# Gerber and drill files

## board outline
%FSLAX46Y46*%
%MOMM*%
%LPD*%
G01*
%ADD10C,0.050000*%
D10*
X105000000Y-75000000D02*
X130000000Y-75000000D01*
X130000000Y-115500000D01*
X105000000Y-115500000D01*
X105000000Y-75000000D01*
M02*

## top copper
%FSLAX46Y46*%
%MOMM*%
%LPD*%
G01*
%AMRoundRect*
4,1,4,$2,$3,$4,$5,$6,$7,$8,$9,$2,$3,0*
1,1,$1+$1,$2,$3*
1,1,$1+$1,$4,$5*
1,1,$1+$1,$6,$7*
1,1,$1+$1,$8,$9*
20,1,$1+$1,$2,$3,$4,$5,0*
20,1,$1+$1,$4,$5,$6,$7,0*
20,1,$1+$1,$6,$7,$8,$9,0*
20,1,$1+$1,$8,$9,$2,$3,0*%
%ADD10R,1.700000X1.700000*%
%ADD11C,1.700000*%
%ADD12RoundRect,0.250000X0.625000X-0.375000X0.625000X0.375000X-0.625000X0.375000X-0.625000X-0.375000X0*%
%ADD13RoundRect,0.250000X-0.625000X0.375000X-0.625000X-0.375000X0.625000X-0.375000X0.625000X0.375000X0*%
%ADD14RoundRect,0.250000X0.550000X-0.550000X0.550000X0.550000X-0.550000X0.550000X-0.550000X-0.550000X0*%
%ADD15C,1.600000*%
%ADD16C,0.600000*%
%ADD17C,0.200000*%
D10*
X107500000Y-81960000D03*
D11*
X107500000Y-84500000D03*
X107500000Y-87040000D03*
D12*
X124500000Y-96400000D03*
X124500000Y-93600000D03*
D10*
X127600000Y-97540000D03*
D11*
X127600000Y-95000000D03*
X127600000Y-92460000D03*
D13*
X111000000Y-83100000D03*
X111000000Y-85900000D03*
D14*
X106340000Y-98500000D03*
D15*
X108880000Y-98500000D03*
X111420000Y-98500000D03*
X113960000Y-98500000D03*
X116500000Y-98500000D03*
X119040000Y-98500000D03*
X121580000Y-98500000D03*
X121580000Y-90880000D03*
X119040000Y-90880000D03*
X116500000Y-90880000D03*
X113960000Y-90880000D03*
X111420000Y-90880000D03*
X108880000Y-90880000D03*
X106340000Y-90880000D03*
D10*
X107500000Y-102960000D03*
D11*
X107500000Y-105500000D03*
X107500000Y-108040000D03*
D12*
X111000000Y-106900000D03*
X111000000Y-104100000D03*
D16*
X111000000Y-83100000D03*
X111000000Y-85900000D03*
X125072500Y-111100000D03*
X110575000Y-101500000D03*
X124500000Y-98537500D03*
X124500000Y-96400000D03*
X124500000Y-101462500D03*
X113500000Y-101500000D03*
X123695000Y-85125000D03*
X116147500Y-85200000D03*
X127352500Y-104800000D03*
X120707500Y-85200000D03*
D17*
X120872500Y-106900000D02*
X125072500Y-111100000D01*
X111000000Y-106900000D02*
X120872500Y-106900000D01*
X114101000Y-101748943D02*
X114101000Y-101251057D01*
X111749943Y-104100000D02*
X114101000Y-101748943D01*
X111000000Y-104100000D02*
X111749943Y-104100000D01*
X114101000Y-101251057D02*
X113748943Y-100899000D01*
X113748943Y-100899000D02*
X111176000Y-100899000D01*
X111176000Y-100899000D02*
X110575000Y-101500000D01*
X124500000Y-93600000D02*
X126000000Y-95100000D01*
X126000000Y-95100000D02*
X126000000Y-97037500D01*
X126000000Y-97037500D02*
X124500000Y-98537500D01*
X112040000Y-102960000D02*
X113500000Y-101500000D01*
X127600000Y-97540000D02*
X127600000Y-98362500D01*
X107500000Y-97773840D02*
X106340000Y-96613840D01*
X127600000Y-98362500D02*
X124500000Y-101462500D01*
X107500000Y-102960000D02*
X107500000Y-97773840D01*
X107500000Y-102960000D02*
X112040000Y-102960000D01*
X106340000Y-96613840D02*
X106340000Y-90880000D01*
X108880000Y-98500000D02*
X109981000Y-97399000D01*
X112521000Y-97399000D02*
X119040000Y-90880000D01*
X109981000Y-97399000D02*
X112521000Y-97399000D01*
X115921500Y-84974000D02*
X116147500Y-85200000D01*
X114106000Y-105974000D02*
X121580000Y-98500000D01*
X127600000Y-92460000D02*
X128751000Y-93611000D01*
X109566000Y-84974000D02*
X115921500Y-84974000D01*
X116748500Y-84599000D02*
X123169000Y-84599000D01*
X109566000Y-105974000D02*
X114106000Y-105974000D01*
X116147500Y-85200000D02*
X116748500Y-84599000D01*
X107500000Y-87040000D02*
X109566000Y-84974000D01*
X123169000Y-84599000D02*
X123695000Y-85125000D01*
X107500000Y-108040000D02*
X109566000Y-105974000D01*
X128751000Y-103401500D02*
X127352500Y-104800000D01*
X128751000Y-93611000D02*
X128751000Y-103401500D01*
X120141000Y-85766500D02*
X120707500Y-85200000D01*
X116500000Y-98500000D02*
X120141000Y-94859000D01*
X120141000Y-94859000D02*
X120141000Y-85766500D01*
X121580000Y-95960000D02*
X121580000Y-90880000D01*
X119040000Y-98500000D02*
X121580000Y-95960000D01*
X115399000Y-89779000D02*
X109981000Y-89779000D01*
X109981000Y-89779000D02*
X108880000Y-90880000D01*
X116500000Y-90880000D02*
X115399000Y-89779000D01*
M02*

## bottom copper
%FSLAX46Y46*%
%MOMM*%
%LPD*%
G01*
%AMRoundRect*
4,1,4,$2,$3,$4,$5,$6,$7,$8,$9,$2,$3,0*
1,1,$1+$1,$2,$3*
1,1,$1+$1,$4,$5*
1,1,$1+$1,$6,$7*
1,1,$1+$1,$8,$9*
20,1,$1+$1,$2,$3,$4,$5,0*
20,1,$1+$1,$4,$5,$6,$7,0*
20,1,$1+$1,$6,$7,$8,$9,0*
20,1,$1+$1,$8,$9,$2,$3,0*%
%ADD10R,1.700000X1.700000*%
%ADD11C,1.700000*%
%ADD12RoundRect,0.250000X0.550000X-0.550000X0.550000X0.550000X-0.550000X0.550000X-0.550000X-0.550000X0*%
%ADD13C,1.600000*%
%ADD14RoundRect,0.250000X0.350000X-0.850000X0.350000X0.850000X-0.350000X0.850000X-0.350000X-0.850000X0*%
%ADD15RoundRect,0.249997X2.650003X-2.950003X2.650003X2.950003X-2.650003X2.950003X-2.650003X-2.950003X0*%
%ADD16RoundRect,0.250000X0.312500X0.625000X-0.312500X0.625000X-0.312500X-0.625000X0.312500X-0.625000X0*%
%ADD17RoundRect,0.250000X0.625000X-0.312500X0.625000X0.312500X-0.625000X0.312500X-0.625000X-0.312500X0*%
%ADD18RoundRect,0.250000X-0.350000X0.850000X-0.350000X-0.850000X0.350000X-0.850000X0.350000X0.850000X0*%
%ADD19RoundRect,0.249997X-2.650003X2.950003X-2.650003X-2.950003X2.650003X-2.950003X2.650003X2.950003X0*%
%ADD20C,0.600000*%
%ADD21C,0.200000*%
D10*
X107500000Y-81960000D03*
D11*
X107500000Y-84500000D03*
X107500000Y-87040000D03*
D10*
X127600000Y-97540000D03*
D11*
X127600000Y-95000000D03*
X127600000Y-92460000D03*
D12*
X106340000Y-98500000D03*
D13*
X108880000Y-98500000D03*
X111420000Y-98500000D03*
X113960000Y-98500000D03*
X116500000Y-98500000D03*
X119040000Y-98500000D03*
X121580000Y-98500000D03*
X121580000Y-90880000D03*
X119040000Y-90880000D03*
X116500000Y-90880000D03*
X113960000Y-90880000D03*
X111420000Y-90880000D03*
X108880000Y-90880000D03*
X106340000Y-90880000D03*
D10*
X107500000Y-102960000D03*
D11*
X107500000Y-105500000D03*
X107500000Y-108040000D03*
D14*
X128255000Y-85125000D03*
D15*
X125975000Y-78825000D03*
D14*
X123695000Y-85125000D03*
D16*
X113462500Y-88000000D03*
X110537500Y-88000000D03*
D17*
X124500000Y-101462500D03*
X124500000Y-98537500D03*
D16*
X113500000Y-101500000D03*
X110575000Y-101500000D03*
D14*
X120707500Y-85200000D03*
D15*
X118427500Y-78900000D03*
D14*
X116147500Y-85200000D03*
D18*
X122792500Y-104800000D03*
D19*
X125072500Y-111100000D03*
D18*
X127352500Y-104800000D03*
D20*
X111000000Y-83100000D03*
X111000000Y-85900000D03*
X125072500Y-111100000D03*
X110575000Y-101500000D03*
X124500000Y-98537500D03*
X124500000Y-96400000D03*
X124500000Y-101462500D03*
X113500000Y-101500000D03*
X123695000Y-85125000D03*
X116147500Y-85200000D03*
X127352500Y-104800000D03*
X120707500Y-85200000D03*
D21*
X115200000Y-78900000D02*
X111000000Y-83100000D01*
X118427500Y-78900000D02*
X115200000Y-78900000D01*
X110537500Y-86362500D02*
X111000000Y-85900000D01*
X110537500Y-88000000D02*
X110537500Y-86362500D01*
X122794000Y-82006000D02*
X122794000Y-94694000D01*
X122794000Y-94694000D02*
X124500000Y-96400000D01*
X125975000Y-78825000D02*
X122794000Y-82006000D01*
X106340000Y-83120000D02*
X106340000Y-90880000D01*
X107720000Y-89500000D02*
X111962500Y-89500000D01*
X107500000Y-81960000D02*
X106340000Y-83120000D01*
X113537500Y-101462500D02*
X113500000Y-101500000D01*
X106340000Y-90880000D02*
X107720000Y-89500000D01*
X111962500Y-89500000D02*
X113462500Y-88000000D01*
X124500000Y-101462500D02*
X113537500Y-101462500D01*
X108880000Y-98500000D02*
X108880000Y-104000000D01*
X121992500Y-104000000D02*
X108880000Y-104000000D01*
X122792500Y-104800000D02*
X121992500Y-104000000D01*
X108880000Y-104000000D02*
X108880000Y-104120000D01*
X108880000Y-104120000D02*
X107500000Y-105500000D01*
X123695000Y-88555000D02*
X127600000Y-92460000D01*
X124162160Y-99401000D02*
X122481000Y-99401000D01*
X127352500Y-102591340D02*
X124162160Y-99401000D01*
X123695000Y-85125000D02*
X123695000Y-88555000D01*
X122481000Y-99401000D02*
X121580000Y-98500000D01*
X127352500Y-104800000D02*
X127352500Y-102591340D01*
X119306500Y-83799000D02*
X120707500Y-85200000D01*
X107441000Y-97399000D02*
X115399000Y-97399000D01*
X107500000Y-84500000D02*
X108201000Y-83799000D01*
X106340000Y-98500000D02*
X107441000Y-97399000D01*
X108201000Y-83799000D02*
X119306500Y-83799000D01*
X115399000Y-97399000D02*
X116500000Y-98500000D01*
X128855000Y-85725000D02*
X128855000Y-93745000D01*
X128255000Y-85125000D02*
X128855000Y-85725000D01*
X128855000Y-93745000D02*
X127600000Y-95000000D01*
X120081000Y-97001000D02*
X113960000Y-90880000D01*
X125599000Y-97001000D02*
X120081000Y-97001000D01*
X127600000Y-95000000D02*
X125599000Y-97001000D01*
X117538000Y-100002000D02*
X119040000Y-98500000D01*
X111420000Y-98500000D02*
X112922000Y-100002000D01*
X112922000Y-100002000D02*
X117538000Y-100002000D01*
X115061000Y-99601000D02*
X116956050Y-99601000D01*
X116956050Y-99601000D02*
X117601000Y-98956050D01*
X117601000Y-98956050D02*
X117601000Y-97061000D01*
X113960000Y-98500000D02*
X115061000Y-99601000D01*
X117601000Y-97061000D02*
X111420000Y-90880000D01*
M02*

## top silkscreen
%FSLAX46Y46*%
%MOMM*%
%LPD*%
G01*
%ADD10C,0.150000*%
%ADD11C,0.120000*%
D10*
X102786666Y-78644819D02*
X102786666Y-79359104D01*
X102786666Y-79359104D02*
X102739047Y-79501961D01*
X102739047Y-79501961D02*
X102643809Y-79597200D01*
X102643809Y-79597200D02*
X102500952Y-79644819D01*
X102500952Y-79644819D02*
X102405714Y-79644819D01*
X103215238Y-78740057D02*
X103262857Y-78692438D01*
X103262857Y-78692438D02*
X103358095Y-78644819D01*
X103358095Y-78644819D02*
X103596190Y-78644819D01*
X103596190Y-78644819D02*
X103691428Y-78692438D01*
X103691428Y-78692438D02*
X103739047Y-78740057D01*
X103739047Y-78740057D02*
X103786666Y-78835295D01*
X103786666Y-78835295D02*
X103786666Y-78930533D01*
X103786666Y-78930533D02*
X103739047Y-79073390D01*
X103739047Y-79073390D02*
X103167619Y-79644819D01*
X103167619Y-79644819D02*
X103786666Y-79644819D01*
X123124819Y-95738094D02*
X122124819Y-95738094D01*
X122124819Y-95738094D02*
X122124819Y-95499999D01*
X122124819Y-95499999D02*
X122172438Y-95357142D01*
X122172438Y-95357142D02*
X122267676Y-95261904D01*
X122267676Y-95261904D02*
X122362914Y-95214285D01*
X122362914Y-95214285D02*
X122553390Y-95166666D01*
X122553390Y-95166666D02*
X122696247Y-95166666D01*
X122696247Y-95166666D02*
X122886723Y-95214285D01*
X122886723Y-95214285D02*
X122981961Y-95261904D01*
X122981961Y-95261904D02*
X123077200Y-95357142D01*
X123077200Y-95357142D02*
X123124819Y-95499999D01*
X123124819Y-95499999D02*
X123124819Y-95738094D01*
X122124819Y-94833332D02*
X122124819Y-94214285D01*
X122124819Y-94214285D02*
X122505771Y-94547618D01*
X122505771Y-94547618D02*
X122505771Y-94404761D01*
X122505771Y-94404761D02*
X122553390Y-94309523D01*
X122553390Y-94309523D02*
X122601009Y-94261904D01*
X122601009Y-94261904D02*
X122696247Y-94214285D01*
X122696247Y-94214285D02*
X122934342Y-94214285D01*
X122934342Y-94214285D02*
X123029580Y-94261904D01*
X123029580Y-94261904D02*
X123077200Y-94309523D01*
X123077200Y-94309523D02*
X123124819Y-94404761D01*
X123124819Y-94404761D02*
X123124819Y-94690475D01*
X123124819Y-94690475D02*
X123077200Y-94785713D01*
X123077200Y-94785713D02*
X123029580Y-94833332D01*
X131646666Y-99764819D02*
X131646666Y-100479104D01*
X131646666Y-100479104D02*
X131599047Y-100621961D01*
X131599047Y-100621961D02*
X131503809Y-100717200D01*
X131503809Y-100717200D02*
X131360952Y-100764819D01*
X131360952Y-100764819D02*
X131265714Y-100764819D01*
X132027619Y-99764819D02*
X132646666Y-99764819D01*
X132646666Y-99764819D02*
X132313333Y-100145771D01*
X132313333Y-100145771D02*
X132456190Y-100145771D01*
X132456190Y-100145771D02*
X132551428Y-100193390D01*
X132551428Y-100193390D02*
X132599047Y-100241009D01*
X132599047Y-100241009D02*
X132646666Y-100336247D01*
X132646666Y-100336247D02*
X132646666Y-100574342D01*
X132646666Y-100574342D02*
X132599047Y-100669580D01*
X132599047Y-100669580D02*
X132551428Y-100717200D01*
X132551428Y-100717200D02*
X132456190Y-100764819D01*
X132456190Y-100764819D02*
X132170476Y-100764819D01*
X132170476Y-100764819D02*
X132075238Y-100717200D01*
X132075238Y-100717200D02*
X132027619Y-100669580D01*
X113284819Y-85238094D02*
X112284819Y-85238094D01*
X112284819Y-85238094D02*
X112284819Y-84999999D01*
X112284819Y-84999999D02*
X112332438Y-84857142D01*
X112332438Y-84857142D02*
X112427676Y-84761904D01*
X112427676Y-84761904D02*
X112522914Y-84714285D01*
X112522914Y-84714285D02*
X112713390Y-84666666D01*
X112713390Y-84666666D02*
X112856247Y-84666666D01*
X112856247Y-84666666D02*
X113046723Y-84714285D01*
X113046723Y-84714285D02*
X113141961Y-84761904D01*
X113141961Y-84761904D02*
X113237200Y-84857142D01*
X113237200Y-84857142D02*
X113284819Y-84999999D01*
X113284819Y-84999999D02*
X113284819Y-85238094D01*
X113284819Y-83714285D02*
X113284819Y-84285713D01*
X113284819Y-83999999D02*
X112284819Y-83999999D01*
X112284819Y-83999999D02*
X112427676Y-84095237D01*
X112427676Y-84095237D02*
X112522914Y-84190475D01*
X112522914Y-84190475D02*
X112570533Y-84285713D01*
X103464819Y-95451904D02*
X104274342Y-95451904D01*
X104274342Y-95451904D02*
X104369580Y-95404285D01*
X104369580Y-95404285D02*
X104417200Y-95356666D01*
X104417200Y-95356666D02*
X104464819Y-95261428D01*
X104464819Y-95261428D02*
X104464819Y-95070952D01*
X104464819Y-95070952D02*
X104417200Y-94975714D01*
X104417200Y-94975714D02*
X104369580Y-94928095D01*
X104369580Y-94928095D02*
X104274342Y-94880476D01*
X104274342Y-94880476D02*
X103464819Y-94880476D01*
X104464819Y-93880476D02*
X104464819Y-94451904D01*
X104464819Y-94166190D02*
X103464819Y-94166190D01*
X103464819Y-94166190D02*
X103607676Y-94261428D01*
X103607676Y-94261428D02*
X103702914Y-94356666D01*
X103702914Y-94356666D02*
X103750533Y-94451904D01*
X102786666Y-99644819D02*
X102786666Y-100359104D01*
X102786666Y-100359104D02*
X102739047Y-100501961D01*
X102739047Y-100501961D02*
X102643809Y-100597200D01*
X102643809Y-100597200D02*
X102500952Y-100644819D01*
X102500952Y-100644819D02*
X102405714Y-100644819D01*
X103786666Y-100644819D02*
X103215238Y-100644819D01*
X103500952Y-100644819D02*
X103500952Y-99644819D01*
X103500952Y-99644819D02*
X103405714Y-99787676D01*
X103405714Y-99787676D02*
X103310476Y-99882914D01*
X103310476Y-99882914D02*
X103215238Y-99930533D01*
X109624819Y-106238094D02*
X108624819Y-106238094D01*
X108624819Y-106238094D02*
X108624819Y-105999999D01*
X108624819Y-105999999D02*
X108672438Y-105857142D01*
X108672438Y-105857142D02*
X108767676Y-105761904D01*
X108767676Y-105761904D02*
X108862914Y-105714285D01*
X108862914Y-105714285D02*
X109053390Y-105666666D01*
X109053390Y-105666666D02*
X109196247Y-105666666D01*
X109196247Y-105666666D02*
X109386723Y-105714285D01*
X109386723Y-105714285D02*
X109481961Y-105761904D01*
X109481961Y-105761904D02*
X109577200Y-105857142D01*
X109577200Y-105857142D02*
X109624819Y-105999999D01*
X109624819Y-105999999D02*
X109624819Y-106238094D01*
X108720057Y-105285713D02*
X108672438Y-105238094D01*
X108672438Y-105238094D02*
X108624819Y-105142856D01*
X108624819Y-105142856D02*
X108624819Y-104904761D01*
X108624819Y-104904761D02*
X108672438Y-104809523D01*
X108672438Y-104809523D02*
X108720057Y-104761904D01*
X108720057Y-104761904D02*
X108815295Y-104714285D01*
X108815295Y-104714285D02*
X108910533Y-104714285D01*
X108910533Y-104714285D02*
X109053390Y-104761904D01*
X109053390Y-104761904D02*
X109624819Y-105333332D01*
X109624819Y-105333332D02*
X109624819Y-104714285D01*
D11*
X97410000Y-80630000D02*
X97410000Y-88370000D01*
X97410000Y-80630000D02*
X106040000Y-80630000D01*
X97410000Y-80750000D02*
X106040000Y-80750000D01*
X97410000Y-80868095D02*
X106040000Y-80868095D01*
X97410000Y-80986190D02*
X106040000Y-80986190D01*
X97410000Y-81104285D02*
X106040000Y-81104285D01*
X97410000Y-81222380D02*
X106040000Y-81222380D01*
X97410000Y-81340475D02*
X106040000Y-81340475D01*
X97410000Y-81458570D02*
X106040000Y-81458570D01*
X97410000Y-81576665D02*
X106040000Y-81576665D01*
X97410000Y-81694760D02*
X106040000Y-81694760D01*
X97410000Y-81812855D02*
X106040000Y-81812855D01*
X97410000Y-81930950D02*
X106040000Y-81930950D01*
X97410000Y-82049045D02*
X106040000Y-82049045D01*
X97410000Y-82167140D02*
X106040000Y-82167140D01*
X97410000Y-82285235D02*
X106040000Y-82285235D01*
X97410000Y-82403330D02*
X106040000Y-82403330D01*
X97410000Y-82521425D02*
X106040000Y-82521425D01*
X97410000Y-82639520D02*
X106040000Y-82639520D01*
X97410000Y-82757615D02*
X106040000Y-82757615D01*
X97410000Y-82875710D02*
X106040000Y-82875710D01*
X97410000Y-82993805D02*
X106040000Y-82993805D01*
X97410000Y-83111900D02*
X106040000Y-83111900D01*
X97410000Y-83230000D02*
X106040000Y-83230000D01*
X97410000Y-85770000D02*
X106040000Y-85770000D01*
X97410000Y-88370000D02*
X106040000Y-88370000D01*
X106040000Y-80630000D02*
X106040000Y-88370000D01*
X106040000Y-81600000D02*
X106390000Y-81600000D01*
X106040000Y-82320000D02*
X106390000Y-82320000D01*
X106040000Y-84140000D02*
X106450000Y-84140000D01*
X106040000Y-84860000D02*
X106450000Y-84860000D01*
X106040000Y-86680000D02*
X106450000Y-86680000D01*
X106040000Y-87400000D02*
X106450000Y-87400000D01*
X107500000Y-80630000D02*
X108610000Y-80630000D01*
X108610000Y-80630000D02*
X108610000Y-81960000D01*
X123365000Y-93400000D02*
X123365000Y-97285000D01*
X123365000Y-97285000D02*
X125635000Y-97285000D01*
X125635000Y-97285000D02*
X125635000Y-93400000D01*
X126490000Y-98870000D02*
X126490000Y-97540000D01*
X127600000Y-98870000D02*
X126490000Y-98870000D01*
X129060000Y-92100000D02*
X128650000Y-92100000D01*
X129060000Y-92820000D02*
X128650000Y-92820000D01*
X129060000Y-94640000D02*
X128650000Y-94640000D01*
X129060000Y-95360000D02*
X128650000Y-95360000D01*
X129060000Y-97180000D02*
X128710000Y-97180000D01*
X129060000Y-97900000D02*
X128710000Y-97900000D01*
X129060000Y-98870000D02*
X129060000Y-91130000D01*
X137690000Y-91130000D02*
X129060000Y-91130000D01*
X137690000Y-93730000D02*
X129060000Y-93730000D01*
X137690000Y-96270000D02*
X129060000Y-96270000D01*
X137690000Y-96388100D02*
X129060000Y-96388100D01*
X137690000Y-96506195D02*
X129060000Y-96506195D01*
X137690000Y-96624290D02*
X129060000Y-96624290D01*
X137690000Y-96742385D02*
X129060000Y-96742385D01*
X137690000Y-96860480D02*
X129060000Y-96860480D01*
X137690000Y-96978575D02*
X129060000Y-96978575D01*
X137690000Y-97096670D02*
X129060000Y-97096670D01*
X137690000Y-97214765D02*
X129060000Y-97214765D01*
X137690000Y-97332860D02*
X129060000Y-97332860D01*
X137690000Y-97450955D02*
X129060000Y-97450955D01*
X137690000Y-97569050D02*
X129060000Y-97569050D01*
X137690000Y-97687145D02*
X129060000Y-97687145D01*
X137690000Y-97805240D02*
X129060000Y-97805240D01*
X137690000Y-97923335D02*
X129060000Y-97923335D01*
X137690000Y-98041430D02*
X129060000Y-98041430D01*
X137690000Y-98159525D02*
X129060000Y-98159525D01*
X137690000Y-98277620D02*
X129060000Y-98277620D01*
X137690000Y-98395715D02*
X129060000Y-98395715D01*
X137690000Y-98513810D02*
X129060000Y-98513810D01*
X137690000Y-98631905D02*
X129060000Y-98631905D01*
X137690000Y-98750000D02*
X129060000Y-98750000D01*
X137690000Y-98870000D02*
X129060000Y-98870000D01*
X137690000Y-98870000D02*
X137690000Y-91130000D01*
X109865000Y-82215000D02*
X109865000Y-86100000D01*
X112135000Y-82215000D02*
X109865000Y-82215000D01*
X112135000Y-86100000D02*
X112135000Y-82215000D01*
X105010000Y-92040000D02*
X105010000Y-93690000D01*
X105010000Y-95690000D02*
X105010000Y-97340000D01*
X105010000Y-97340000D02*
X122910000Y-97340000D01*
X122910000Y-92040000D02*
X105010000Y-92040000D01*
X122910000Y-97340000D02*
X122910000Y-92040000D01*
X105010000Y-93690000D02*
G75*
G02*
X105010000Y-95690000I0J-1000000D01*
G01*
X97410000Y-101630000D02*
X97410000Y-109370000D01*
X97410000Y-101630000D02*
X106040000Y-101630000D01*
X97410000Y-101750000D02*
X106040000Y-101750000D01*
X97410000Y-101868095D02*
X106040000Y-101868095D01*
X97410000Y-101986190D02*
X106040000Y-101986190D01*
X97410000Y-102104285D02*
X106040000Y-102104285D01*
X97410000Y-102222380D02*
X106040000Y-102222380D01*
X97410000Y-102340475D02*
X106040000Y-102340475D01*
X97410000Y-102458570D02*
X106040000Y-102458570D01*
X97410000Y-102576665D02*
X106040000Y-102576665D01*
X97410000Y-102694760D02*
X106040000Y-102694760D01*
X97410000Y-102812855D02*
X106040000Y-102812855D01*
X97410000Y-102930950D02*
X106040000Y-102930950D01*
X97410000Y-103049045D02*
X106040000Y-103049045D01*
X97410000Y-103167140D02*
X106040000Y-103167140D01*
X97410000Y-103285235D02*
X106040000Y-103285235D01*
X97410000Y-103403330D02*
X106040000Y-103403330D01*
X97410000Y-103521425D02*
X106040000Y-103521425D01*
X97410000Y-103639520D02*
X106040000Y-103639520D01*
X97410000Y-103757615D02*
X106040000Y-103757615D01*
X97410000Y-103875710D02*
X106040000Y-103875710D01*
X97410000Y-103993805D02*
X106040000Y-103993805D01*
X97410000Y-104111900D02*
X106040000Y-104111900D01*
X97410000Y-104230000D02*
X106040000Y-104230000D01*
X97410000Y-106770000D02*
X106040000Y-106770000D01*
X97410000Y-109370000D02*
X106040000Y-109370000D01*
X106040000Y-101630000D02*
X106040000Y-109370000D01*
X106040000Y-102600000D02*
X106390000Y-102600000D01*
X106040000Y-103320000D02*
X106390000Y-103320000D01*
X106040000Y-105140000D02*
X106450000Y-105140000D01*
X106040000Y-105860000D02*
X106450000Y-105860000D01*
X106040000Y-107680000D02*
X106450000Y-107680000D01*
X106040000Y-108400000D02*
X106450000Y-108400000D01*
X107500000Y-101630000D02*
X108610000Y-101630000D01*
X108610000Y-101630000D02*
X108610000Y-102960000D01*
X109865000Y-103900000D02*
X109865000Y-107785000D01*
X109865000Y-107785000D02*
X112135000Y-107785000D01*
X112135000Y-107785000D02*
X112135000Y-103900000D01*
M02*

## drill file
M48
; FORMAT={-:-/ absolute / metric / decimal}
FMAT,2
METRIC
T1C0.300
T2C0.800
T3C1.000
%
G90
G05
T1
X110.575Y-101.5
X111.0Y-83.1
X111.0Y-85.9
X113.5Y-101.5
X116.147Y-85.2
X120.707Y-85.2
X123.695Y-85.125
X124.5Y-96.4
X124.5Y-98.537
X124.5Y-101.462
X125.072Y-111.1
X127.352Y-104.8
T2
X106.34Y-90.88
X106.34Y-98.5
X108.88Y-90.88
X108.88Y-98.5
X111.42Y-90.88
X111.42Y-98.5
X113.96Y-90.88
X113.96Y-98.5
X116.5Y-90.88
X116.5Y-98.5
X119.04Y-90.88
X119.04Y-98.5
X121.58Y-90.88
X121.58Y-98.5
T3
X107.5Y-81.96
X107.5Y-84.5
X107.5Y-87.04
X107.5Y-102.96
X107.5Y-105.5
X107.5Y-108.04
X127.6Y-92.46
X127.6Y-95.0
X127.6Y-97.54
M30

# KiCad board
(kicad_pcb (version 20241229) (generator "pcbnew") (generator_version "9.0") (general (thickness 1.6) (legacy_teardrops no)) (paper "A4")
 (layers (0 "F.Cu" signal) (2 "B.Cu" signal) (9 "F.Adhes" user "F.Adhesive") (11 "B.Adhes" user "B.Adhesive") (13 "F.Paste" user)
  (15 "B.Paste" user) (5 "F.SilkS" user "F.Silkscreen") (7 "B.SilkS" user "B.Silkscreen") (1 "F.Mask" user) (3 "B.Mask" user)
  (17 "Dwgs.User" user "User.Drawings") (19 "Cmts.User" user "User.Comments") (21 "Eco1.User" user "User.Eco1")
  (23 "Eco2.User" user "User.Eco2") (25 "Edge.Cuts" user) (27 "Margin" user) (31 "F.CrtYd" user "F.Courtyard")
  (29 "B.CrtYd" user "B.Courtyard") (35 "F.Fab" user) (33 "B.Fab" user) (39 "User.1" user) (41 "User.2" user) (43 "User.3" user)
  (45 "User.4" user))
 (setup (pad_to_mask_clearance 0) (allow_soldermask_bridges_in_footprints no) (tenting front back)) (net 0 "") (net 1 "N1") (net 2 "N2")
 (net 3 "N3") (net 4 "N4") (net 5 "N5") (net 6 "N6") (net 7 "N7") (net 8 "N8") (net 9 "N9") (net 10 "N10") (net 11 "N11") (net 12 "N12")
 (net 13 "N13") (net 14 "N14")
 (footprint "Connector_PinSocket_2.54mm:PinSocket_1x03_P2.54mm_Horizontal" (layer "F.Cu") (at 107.5 81.96)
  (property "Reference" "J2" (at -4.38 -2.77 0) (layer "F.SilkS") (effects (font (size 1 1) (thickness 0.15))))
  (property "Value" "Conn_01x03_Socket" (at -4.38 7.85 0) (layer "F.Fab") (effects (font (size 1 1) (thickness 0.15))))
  (fp_line (start -10.09 -1.33) (end -10.09 6.41) (stroke (width 0.12) (type solid)) (layer "F.SilkS"))
  (fp_line (start -10.09 -1.33) (end -1.46 -1.33) (stroke (width 0.12) (type solid)) (layer "F.SilkS"))
  (fp_line (start -10.09 -1.21) (end -1.46 -1.21) (stroke (width 0.12) (type solid)) (layer "F.SilkS"))
  (fp_line (start -10.09 -1.091905) (end -1.46 -1.091905) (stroke (width 0.12) (type solid)) (layer "F.SilkS"))
  (fp_line (start -10.09 -0.97381) (end -1.46 -0.97381) (stroke (width 0.12) (type solid)) (layer "F.SilkS"))
  (fp_line (start -10.09 -0.855715) (end -1.46 -0.855715) (stroke (width 0.12) (type solid)) (layer "F.SilkS"))
  (fp_line (start -10.09 -0.73762) (end -1.46 -0.73762) (stroke (width 0.12) (type solid)) (layer "F.SilkS"))
  (fp_line (start -10.09 -0.619525) (end -1.46 -0.619525) (stroke (width 0.12) (type solid)) (layer "F.SilkS"))
  (fp_line (start -10.09 -0.50143) (end -1.46 -0.50143) (stroke (width 0.12) (type solid)) (layer "F.SilkS"))
  (fp_line (start -10.09 -0.383335) (end -1.46 -0.383335) (stroke (width 0.12) (type solid)) (layer "F.SilkS"))
  (fp_line (start -10.09 -0.26524) (end -1.46 -0.26524) (stroke (width 0.12) (type solid)) (layer "F.SilkS"))
  (fp_line (start -10.09 -0.147145) (end -1.46 -0.147145) (stroke (width 0.12) (type solid)) (layer "F.SilkS"))
  (fp_line (start -10.09 -0.02905) (end -1.46 -0.02905) (stroke (width 0.12) (type solid)) (layer "F.SilkS"))
  (fp_line (start -10.09 0.089045) (end -1.46 0.089045) (stroke (width 0.12) (type solid)) (layer "F.SilkS"))
  (fp_line (start -10.09 0.20714) (end -1.46 0.20714) (stroke (width 0.12) (type solid)) (layer "F.SilkS"))
  (fp_line (start -10.09 0.325235) (end -1.46 0.325235) (stroke (width 0.12) (type solid)) (layer "F.SilkS"))
  (fp_line (start -10.09 0.44333) (end -1.46 0.44333) (stroke (width 0.12) (type solid)) (layer "F.SilkS"))
  (fp_line (start -10.09 0.561425) (end -1.46 0.561425) (stroke (width 0.12) (type solid)) (layer "F.SilkS"))
  (fp_line (start -10.09 0.67952) (end -1.46 0.67952) (stroke (width 0.12) (type solid)) (layer "F.SilkS"))
  (fp_line (start -10.09 0.797615) (end -1.46 0.797615) (stroke (width 0.12) (type solid)) (layer "F.SilkS"))
  (fp_line (start -10.09 0.91571) (end -1.46 0.91571) (stroke (width 0.12) (type solid)) (layer "F.SilkS"))
  (fp_line (start -10.09 1.033805) (end -1.46 1.033805) (stroke (width 0.12) (type solid)) (layer "F.SilkS"))
  (fp_line (start -10.09 1.1519) (end -1.46 1.1519) (stroke (width 0.12) (type solid)) (layer "F.SilkS"))
  (fp_line (start -10.09 1.27) (end -1.46 1.27) (stroke (width 0.12) (type solid)) (layer "F.SilkS"))
  (fp_line (start -10.09 3.81) (end -1.46 3.81) (stroke (width 0.12) (type solid)) (layer "F.SilkS"))
  (fp_line (start -10.09 6.41) (end -1.46 6.41) (stroke (width 0.12) (type solid)) (layer "F.SilkS"))
  (fp_line (start -1.46 -1.33) (end -1.46 6.41) (stroke (width 0.12) (type solid)) (layer "F.SilkS"))
  (fp_line (start -1.46 -0.36) (end -1.11 -0.36) (stroke (width 0.12) (type solid)) (layer "F.SilkS"))
  (fp_line (start -1.46 0.36) (end -1.11 0.36) (stroke (width 0.12) (type solid)) (layer "F.SilkS"))
  (fp_line (start -1.46 2.18) (end -1.05 2.18) (stroke (width 0.12) (type solid)) (layer "F.SilkS"))
  (fp_line (start -1.46 2.9) (end -1.05 2.9) (stroke (width 0.12) (type solid)) (layer "F.SilkS"))
  (fp_line (start -1.46 4.72) (end -1.05 4.72) (stroke (width 0.12) (type solid)) (layer "F.SilkS"))
  (fp_line (start -1.46 5.44) (end -1.05 5.44) (stroke (width 0.12) (type solid)) (layer "F.SilkS"))
  (fp_line (start 0 -1.33) (end 1.11 -1.33) (stroke (width 0.12) (type solid)) (layer "F.SilkS"))
  (fp_line (start 1.11 -1.33) (end 1.11 0) (stroke (width 0.12) (type solid)) (layer "F.SilkS"))
  (pad "1" thru_hole rect (at 0 0) (size 1.7 1.7) (drill 1) (layers "*.Cu" "*.Mask") (remove_unused_layers no) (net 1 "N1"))
  (pad "2" thru_hole circle (at 0 2.54) (size 1.7 1.7) (drill 1) (layers "*.Cu" "*.Mask") (remove_unused_layers no) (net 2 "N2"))
  (pad "3" thru_hole circle (at 0 5.08) (size 1.7 1.7) (drill 1) (layers "*.Cu" "*.Mask") (remove_unused_layers no) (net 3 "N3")))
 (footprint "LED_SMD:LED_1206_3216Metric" (layer "F.Cu") (at 124.5 95 90)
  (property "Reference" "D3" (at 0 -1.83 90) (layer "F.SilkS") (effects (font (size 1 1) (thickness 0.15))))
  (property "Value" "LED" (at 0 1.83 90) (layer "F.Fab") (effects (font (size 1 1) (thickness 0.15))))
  (fp_line (start 1.6 -1.135) (end -2.285 -1.135) (stroke (width 0.12) (type solid)) (layer "F.SilkS"))
  (fp_line (start -2.285 -1.135) (end -2.285 1.135) (stroke (width 0.12) (type solid)) (layer "F.SilkS"))
  (fp_line (start -2.285 1.135) (end 1.6 1.135) (stroke (width 0.12) (type solid)) (layer "F.SilkS"))
  (pad "1" smd roundrect (at -1.4 0 90) (size 1.25 1.75) (layers "F.Cu" "F.Mask" "F.Paste") (roundrect_rratio 0.2) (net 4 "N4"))
  (pad "2" smd roundrect (at 1.4 0 90) (size 1.25 1.75) (layers "F.Cu" "F.Mask" "F.Paste") (roundrect_rratio 0.2) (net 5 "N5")))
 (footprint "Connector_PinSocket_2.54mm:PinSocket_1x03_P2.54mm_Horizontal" (layer "F.Cu") (at 127.6 97.54 180)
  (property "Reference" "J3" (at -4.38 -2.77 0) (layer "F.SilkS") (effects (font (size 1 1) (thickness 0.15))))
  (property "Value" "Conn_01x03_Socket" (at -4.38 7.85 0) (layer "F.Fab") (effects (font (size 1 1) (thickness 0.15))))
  (fp_line (start 1.11 -1.33) (end 1.11 0) (stroke (width 0.12) (type solid)) (layer "F.SilkS"))
  (fp_line (start 0 -1.33) (end 1.11 -1.33) (stroke (width 0.12) (type solid)) (layer "F.SilkS"))
  (fp_line (start -1.46 5.44) (end -1.05 5.44) (stroke (width 0.12) (type solid)) (layer "F.SilkS"))
  (fp_line (start -1.46 4.72) (end -1.05 4.72) (stroke (width 0.12) (type solid)) (layer "F.SilkS"))
  (fp_line (start -1.46 2.9) (end -1.05 2.9) (stroke (width 0.12) (type solid)) (layer "F.SilkS"))
  (fp_line (start -1.46 2.18) (end -1.05 2.18) (stroke (width 0.12) (type solid)) (layer "F.SilkS"))
  (fp_line (start -1.46 0.36) (end -1.11 0.36) (stroke (width 0.12) (type solid)) (layer "F.SilkS"))
  (fp_line (start -1.46 -0.36) (end -1.11 -0.36) (stroke (width 0.12) (type solid)) (layer "F.SilkS"))
  (fp_line (start -1.46 -1.33) (end -1.46 6.41) (stroke (width 0.12) (type solid)) (layer "F.SilkS"))
  (fp_line (start -10.09 6.41) (end -1.46 6.41) (stroke (width 0.12) (type solid)) (layer "F.SilkS"))
  (fp_line (start -10.09 3.81) (end -1.46 3.81) (stroke (width 0.12) (type solid)) (layer "F.SilkS"))
  (fp_line (start -10.09 1.27) (end -1.46 1.27) (stroke (width 0.12) (type solid)) (layer "F.SilkS"))
  (fp_line (start -10.09 1.1519) (end -1.46 1.1519) (stroke (width 0.12) (type solid)) (layer "F.SilkS"))
  (fp_line (start -10.09 1.033805) (end -1.46 1.033805) (stroke (width 0.12) (type solid)) (layer "F.SilkS"))
  (fp_line (start -10.09 0.91571) (end -1.46 0.91571) (stroke (width 0.12) (type solid)) (layer "F.SilkS"))
  (fp_line (start -10.09 0.797615) (end -1.46 0.797615) (stroke (width 0.12) (type solid)) (layer "F.SilkS"))
  (fp_line (start -10.09 0.67952) (end -1.46 0.67952) (stroke (width 0.12) (type solid)) (layer "F.SilkS"))
  (fp_line (start -10.09 0.561425) (end -1.46 0.561425) (stroke (width 0.12) (type solid)) (layer "F.SilkS"))
  (fp_line (start -10.09 0.44333) (end -1.46 0.44333) (stroke (width 0.12) (type solid)) (layer "F.SilkS"))
  (fp_line (start -10.09 0.325235) (end -1.46 0.325235) (stroke (width 0.12) (type solid)) (layer "F.SilkS"))
  (fp_line (start -10.09 0.20714) (end -1.46 0.20714) (stroke (width 0.12) (type solid)) (layer "F.SilkS"))
  (fp_line (start -10.09 0.089045) (end -1.46 0.089045) (stroke (width 0.12) (type solid)) (layer "F.SilkS"))
  (fp_line (start -10.09 -0.02905) (end -1.46 -0.02905) (stroke (width 0.12) (type solid)) (layer "F.SilkS"))
  (fp_line (start -10.09 -0.147145) (end -1.46 -0.147145) (stroke (width 0.12) (type solid)) (layer "F.SilkS"))
  (fp_line (start -10.09 -0.26524) (end -1.46 -0.26524) (stroke (width 0.12) (type solid)) (layer "F.SilkS"))
  (fp_line (start -10.09 -0.383335) (end -1.46 -0.383335) (stroke (width 0.12) (type solid)) (layer "F.SilkS"))
  (fp_line (start -10.09 -0.50143) (end -1.46 -0.50143) (stroke (width 0.12) (type solid)) (layer "F.SilkS"))
  (fp_line (start -10.09 -0.619525) (end -1.46 -0.619525) (stroke (width 0.12) (type solid)) (layer "F.SilkS"))
  (fp_line (start -10.09 -0.73762) (end -1.46 -0.73762) (stroke (width 0.12) (type solid)) (layer "F.SilkS"))
  (fp_line (start -10.09 -0.855715) (end -1.46 -0.855715) (stroke (width 0.12) (type solid)) (layer "F.SilkS"))
  (fp_line (start -10.09 -0.97381) (end -1.46 -0.97381) (stroke (width 0.12) (type solid)) (layer "F.SilkS"))
  (fp_line (start -10.09 -1.091905) (end -1.46 -1.091905) (stroke (width 0.12) (type solid)) (layer "F.SilkS"))
  (fp_line (start -10.09 -1.21) (end -1.46 -1.21) (stroke (width 0.12) (type solid)) (layer "F.SilkS"))
  (fp_line (start -10.09 -1.33) (end -1.46 -1.33) (stroke (width 0.12) (type solid)) (layer "F.SilkS"))
  (fp_line (start -10.09 -1.33) (end -10.09 6.41) (stroke (width 0.12) (type solid)) (layer "F.SilkS"))
  (pad "1" thru_hole rect (at 0 0 180) (size 1.7 1.7) (drill 1) (layers "*.Cu" "*.Mask") (remove_unused_layers no) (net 1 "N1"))
  (pad "2" thru_hole circle (at 0 2.54 180) (size 1.7 1.7) (drill 1) (layers "*.Cu" "*.Mask") (remove_unused_layers no) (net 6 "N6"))
  (pad "3" thru_hole circle (at 0 5.08 180) (size 1.7 1.7) (drill 1) (layers "*.Cu" "*.Mask") (remove_unused_layers no) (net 3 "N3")))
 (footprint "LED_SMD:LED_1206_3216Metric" (layer "F.Cu") (at 111 84.5 -90)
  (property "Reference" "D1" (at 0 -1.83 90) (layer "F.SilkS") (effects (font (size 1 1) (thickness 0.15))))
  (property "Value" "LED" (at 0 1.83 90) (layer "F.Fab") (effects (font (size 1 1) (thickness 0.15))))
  (fp_line (start -2.285 1.135) (end 1.6 1.135) (stroke (width 0.12) (type solid)) (layer "F.SilkS"))
  (fp_line (start -2.285 -1.135) (end -2.285 1.135) (stroke (width 0.12) (type solid)) (layer "F.SilkS"))
  (fp_line (start 1.6 -1.135) (end -2.285 -1.135) (stroke (width 0.12) (type solid)) (layer "F.SilkS"))
  (pad "1" smd roundrect (at -1.4 0 270) (size 1.25 1.75) (layers "F.Cu" "F.Mask" "F.Paste") (roundrect_rratio 0.2) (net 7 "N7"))
  (pad "2" smd roundrect (at 1.4 0 270) (size 1.25 1.75) (layers "F.Cu" "F.Mask" "F.Paste") (roundrect_rratio 0.2) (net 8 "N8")))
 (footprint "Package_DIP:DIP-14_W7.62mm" (layer "F.Cu") (at 106.34 98.5 90)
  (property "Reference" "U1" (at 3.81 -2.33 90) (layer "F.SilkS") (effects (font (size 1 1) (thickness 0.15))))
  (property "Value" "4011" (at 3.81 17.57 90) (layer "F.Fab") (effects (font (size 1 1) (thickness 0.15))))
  (fp_line (start 6.46 -1.33) (end 4.81 -1.33) (stroke (width 0.12) (type solid)) (layer "F.SilkS"))
  (fp_line (start 2.81 -1.33) (end 1.16 -1.33) (stroke (width 0.12) (type solid)) (layer "F.SilkS"))
  (fp_line (start 1.16 -1.33) (end 1.16 16.57) (stroke (width 0.12) (type solid)) (layer "F.SilkS"))
  (fp_line (start 6.46 16.57) (end 6.46 -1.33) (stroke (width 0.12) (type solid)) (layer "F.SilkS"))
  (fp_line (start 1.16 16.57) (end 6.46 16.57) (stroke (width 0.12) (type solid)) (layer "F.SilkS"))
  (fp_arc (start 4.81 -1.33) (mid 3.81 -0.33) (end 2.81 -1.33) (stroke (width 0.12) (type solid)) (layer "F.SilkS"))
  (pad "1" thru_hole roundrect (at 0 0 90) (size 1.6 1.6) (drill 0.8) (layers "*.Cu" "*.Mask") (remove_unused_layers no)
   (roundrect_rratio 0.15625) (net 2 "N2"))
  (pad "2" thru_hole circle (at 0 2.54 90) (size 1.6 1.6) (drill 0.8) (layers "*.Cu" "*.Mask") (remove_unused_layers no) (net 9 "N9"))
  (pad "3" thru_hole circle (at 0 5.08 90) (size 1.6 1.6) (drill 0.8) (layers "*.Cu" "*.Mask") (remove_unused_layers no) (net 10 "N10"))
  (pad "4" thru_hole circle (at 0 7.62 90) (size 1.6 1.6) (drill 0.8) (layers "*.Cu" "*.Mask") (remove_unused_layers no) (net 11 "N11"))
  (pad "5" thru_hole circle (at 0 10.16 90) (size 1.6 1.6) (drill 0.8) (layers "*.Cu" "*.Mask") (remove_unused_layers no) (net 2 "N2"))
  (pad "6" thru_hole circle (at 0 12.7 90) (size 1.6 1.6) (drill 0.8) (layers "*.Cu" "*.Mask") (remove_unused_layers no) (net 10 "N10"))
  (pad "7" thru_hole circle (at 0 15.24 90) (size 1.6 1.6) (drill 0.8) (layers "*.Cu" "*.Mask") (remove_unused_layers no) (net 3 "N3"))
  (pad "8" thru_hole circle (at 7.62 15.24 90) (size 1.6 1.6) (drill 0.8) (layers "*.Cu" "*.Mask") (remove_unused_layers no) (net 10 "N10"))
  (pad "9" thru_hole circle (at 7.62 12.7 90) (size 1.6 1.6) (drill 0.8) (layers "*.Cu" "*.Mask") (remove_unused_layers no) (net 9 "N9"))
  (pad "10" thru_hole circle (at 7.62 10.16 90) (size 1.6 1.6) (drill 0.8) (layers "*.Cu" "*.Mask") (remove_unused_layers no) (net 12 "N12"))
  (pad "11" thru_hole circle (at 7.62 7.62 90) (size 1.6 1.6) (drill 0.8) (layers "*.Cu" "*.Mask") (remove_unused_layers no) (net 6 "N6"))
  (pad "12" thru_hole circle (at 7.62 5.08 90) (size 1.6 1.6) (drill 0.8) (layers "*.Cu" "*.Mask") (remove_unused_layers no) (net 11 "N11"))
  (pad "13" thru_hole circle (at 7.62 2.54 90) (size 1.6 1.6) (drill 0.8) (layers "*.Cu" "*.Mask") (remove_unused_layers no) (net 12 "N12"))
  (pad "14" thru_hole circle (at 7.62 0 90) (size 1.6 1.6) (drill 0.8) (layers "*.Cu" "*.Mask") (remove_unused_layers no) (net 1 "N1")))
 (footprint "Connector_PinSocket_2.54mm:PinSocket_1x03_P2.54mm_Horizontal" (layer "F.Cu") (at 107.5 102.96)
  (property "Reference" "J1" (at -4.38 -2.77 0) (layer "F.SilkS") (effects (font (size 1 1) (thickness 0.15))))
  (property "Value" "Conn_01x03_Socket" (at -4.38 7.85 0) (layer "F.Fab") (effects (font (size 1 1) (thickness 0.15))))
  (fp_line (start -10.09 -1.33) (end -10.09 6.41) (stroke (width 0.12) (type solid)) (layer "F.SilkS"))
  (fp_line (start -10.09 -1.33) (end -1.46 -1.33) (stroke (width 0.12) (type solid)) (layer "F.SilkS"))
  (fp_line (start -10.09 -1.21) (end -1.46 -1.21) (stroke (width 0.12) (type solid)) (layer "F.SilkS"))
  (fp_line (start -10.09 -1.091905) (end -1.46 -1.091905) (stroke (width 0.12) (type solid)) (layer "F.SilkS"))
  (fp_line (start -10.09 -0.97381) (end -1.46 -0.97381) (stroke (width 0.12) (type solid)) (layer "F.SilkS"))
  (fp_line (start -10.09 -0.855715) (end -1.46 -0.855715) (stroke (width 0.12) (type solid)) (layer "F.SilkS"))
  (fp_line (start -10.09 -0.73762) (end -1.46 -0.73762) (stroke (width 0.12) (type solid)) (layer "F.SilkS"))
  (fp_line (start -10.09 -0.619525) (end -1.46 -0.619525) (stroke (width 0.12) (type solid)) (layer "F.SilkS"))
  (fp_line (start -10.09 -0.50143) (end -1.46 -0.50143) (stroke (width 0.12) (type solid)) (layer "F.SilkS"))
  (fp_line (start -10.09 -0.383335) (end -1.46 -0.383335) (stroke (width 0.12) (type solid)) (layer "F.SilkS"))
  (fp_line (start -10.09 -0.26524) (end -1.46 -0.26524) (stroke (width 0.12) (type solid)) (layer "F.SilkS"))
  (fp_line (start -10.09 -0.147145) (end -1.46 -0.147145) (stroke (width 0.12) (type solid)) (layer "F.SilkS"))
  (fp_line (start -10.09 -0.02905) (end -1.46 -0.02905) (stroke (width 0.12) (type solid)) (layer "F.SilkS"))
  (fp_line (start -10.09 0.089045) (end -1.46 0.089045) (stroke (width 0.12) (type solid)) (layer "F.SilkS"))
  (fp_line (start -10.09 0.20714) (end -1.46 0.20714) (stroke (width 0.12) (type solid)) (layer "F.SilkS"))
  (fp_line (start -10.09 0.325235) (end -1.46 0.325235) (stroke (width 0.12) (type solid)) (layer "F.SilkS"))
  (fp_line (start -10.09 0.44333) (end -1.46 0.44333) (stroke (width 0.12) (type solid)) (layer "F.SilkS"))
  (fp_line (start -10.09 0.561425) (end -1.46 0.561425) (stroke (width 0.12) (type solid)) (layer "F.SilkS"))
  (fp_line (start -10.09 0.67952) (end -1.46 0.67952) (stroke (width 0.12) (type solid)) (layer "F.SilkS"))
  (fp_line (start -10.09 0.797615) (end -1.46 0.797615) (stroke (width 0.12) (type solid)) (layer "F.SilkS"))
  (fp_line (start -10.09 0.91571) (end -1.46 0.91571) (stroke (width 0.12) (type solid)) (layer "F.SilkS"))
  (fp_line (start -10.09 1.033805) (end -1.46 1.033805) (stroke (width 0.12) (type solid)) (layer "F.SilkS"))
  (fp_line (start -10.09 1.1519) (end -1.46 1.1519) (stroke (width 0.12) (type solid)) (layer "F.SilkS"))
  (fp_line (start -10.09 1.27) (end -1.46 1.27) (stroke (width 0.12) (type solid)) (layer "F.SilkS"))
  (fp_line (start -10.09 3.81) (end -1.46 3.81) (stroke (width 0.12) (type solid)) (layer "F.SilkS"))
  (fp_line (start -10.09 6.41) (end -1.46 6.41) (stroke (width 0.12) (type solid)) (layer "F.SilkS"))
  (fp_line (start -1.46 -1.33) (end -1.46 6.41) (stroke (width 0.12) (type solid)) (layer "F.SilkS"))
  (fp_line (start -1.46 -0.36) (end -1.11 -0.36) (stroke (width 0.12) (type solid)) (layer "F.SilkS"))
  (fp_line (start -1.46 0.36) (end -1.11 0.36) (stroke (width 0.12) (type solid)) (layer "F.SilkS"))
  (fp_line (start -1.46 2.18) (end -1.05 2.18) (stroke (width 0.12) (type solid)) (layer "F.SilkS"))
  (fp_line (start -1.46 2.9) (end -1.05 2.9) (stroke (width 0.12) (type solid)) (layer "F.SilkS"))
  (fp_line (start -1.46 4.72) (end -1.05 4.72) (stroke (width 0.12) (type solid)) (layer "F.SilkS"))
  (fp_line (start -1.46 5.44) (end -1.05 5.44) (stroke (width 0.12) (type solid)) (layer "F.SilkS"))
  (fp_line (start 0 -1.33) (end 1.11 -1.33) (stroke (width 0.12) (type solid)) (layer "F.SilkS"))
  (fp_line (start 1.11 -1.33) (end 1.11 0) (stroke (width 0.12) (type solid)) (layer "F.SilkS"))
  (pad "1" thru_hole rect (at 0 0) (size 1.7 1.7) (drill 1) (layers "*.Cu" "*.Mask") (remove_unused_layers no) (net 1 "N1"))
  (pad "2" thru_hole circle (at 0 2.54) (size 1.7 1.7) (drill 1) (layers "*.Cu" "*.Mask") (remove_unused_layers no) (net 9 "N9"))
  (pad "3" thru_hole circle (at 0 5.08) (size 1.7 1.7) (drill 1) (layers "*.Cu" "*.Mask") (remove_unused_layers no) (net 3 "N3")))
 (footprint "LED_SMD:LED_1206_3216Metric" (layer "F.Cu") (at 111 105.5 90)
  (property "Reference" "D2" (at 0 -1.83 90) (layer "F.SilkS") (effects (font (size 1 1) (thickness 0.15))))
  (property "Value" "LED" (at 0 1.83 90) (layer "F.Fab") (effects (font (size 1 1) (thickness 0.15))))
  (fp_line (start 1.6 -1.135) (end -2.285 -1.135) (stroke (width 0.12) (type solid)) (layer "F.SilkS"))
  (fp_line (start -2.285 -1.135) (end -2.285 1.135) (stroke (width 0.12) (type solid)) (layer "F.SilkS"))
  (fp_line (start -2.285 1.135) (end 1.6 1.135) (stroke (width 0.12) (type solid)) (layer "F.SilkS"))
  (pad "1" smd roundrect (at -1.4 0 90) (size 1.25 1.75) (layers "F.Cu" "F.Mask" "F.Paste") (roundrect_rratio 0.2) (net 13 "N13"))
  (pad "2" smd roundrect (at 1.4 0 90) (size 1.25 1.75) (layers "F.Cu" "F.Mask" "F.Paste") (roundrect_rratio 0.2) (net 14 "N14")))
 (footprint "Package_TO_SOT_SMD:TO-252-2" (layer "B.Cu") (at 125.975 80.085 90)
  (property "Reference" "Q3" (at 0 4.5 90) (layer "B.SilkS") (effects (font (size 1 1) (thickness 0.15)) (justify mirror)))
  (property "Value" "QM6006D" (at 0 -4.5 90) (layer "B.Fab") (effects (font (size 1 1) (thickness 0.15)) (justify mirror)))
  (pad "" smd roundrect (at -0.415 -1.525 90) (size 3.05 2.75) (layers "B.Paste") (roundrect_rratio 0.090909))
  (pad "" smd roundrect (at -0.415 1.525 90) (size 3.05 2.75) (layers "B.Paste") (roundrect_rratio 0.090909))
  (pad "" smd roundrect (at 2.935 -1.525 90) (size 3.05 2.75) (layers "B.Paste") (roundrect_rratio 0.090909))
  (pad "" smd roundrect (at 2.935 1.525 90) (size 3.05 2.75) (layers "B.Paste") (roundrect_rratio 0.090909))
  (pad "1" smd roundrect (at -5.04 2.28 90) (size 2.2 1.2) (layers "B.Cu" "B.Mask" "B.Paste") (roundrect_rratio 0.208333) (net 6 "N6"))
  (pad "2" smd roundrect (at 1.26 0 90) (size 6.4 5.8) (layers "B.Cu" "B.Mask") (roundrect_rratio 0.043103) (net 4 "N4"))
  (pad "3" smd roundrect (at -5.04 -2.28 90) (size 2.2 1.2) (layers "B.Cu" "B.Mask" "B.Paste") (roundrect_rratio 0.208333) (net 3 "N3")))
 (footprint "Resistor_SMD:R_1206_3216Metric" (layer "B.Cu") (at 112 88 180)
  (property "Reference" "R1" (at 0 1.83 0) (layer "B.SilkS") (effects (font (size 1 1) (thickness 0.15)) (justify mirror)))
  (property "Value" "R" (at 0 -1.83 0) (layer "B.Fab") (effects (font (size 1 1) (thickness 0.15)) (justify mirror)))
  (pad "1" smd roundrect (at -1.4625 0 180) (size 1.125 1.75) (layers "B.Cu" "B.Mask" "B.Paste") (roundrect_rratio 0.222222) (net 1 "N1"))
  (pad "2" smd roundrect (at 1.4625 0 180) (size 1.125 1.75) (layers "B.Cu" "B.Mask" "B.Paste") (roundrect_rratio 0.222222) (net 8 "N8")))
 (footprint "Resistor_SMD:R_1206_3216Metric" (layer "B.Cu") (at 124.5 100 90)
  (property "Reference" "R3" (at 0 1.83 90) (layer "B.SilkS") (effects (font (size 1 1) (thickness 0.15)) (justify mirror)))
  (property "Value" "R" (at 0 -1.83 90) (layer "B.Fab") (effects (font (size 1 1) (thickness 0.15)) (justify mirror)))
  (pad "1" smd roundrect (at -1.4625 0 90) (size 1.125 1.75) (layers "B.Cu" "B.Mask" "B.Paste") (roundrect_rratio 0.222222) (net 1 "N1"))
  (pad "2" smd roundrect (at 1.4625 0 90) (size 1.125 1.75) (layers "B.Cu" "B.Mask" "B.Paste") (roundrect_rratio 0.222222) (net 5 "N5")))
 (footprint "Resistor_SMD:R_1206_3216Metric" (layer "B.Cu") (at 112.0375 101.5 180)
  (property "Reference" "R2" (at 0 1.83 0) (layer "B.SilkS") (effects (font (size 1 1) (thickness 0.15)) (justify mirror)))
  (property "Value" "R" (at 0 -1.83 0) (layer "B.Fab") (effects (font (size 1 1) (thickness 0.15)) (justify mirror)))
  (pad "1" smd roundrect (at -1.4625 0 180) (size 1.125 1.75) (layers "B.Cu" "B.Mask" "B.Paste") (roundrect_rratio 0.222222) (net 1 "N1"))
  (pad "2" smd roundrect (at 1.4625 0 180) (size 1.125 1.75) (layers "B.Cu" "B.Mask" "B.Paste") (roundrect_rratio 0.222222) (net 14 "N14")))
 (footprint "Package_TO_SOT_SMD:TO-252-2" (layer "B.Cu") (at 118.4275 80.16 90)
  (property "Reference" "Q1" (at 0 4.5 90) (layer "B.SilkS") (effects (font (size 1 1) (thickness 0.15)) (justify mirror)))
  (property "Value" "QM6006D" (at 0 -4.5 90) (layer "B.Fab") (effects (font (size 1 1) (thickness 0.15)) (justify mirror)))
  (pad "" smd roundrect (at -0.415 -1.525 90) (size 3.05 2.75) (layers "B.Paste") (roundrect_rratio 0.090909))
  (pad "" smd roundrect (at -0.415 1.525 90) (size 3.05 2.75) (layers "B.Paste") (roundrect_rratio 0.090909))
  (pad "" smd roundrect (at 2.935 -1.525 90) (size 3.05 2.75) (layers "B.Paste") (roundrect_rratio 0.090909))
  (pad "" smd roundrect (at 2.935 1.525 90) (size 3.05 2.75) (layers "B.Paste") (roundrect_rratio 0.090909))
  (pad "1" smd roundrect (at -5.04 2.28 90) (size 2.2 1.2) (layers "B.Cu" "B.Mask" "B.Paste") (roundrect_rratio 0.208333) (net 2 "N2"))
  (pad "2" smd roundrect (at 1.26 0 90) (size 6.4 5.8) (layers "B.Cu" "B.Mask") (roundrect_rratio 0.043103) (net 7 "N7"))
  (pad "3" smd roundrect (at -5.04 -2.28 90) (size 2.2 1.2) (layers "B.Cu" "B.Mask" "B.Paste") (roundrect_rratio 0.208333) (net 3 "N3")))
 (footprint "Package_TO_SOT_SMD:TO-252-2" (layer "B.Cu") (at 125.0725 109.84 -90)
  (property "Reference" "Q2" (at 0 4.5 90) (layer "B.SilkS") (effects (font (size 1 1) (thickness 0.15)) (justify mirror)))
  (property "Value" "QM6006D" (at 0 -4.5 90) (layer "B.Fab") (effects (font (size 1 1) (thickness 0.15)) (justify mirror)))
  (pad "" smd roundrect (at -0.415 -1.525 270) (size 3.05 2.75) (layers "B.Paste") (roundrect_rratio 0.090909))
  (pad "" smd roundrect (at -0.415 1.525 270) (size 3.05 2.75) (layers "B.Paste") (roundrect_rratio 0.090909))
  (pad "" smd roundrect (at 2.935 -1.525 270) (size 3.05 2.75) (layers "B.Paste") (roundrect_rratio 0.090909))
  (pad "" smd roundrect (at 2.935 1.525 270) (size 3.05 2.75) (layers "B.Paste") (roundrect_rratio 0.090909))
  (pad "1" smd roundrect (at -5.04 2.28 270) (size 2.2 1.2) (layers "B.Cu" "B.Mask" "B.Paste") (roundrect_rratio 0.208333) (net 9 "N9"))
  (pad "2" smd roundrect (at 1.26 0 270) (size 6.4 5.8) (layers "B.Cu" "B.Mask") (roundrect_rratio 0.043103) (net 13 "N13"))
  (pad "3" smd roundrect (at -5.04 -2.28 270) (size 2.2 1.2) (layers "B.Cu" "B.Mask" "B.Paste") (roundrect_rratio 0.208333) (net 3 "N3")))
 (gr_rect (start 105 75) (end 130 115.5) (stroke (width 0.05) (type default)) (fill no) (layer "Edge.Cuts"))
 (via (at 111 83.1) (size 0.6) (drill 0.3) (layers "F.Cu" "B.Cu") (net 7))
 (segment (start 115.2 78.9) (end 111 83.1) (width 0.2) (layer "B.Cu") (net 7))
 (segment (start 118.4275 78.9) (end 115.2 78.9) (width 0.2) (layer "B.Cu") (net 7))
 (via (at 111 85.9) (size 0.6) (drill 0.3) (layers "F.Cu" "B.Cu") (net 8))
 (segment (start 110.5375 86.3625) (end 111 85.9) (width 0.2) (layer "B.Cu") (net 8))
 (segment (start 110.5375 88) (end 110.5375 86.3625) (width 0.2) (layer "B.Cu") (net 8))
 (segment (start 120.8725 106.9) (end 125.0725 111.1) (width 0.2) (layer "F.Cu") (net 13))
 (segment (start 111 106.9) (end 120.8725 106.9) (width 0.2) (layer "F.Cu") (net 13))
 (via (at 125.0725 111.1) (size 0.6) (drill 0.3) (layers "F.Cu" "B.Cu") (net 13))
 (segment (start 114.101 101.748943) (end 114.101 101.251057) (width 0.2) (layer "F.Cu") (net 14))
 (segment (start 111.749943 104.1) (end 114.101 101.748943) (width 0.2) (layer "F.Cu") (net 14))
 (segment (start 111 104.1) (end 111.749943 104.1) (width 0.2) (layer "F.Cu") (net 14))
 (segment (start 114.101 101.251057) (end 113.748943 100.899) (width 0.2) (layer "F.Cu") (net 14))
 (segment (start 113.748943 100.899) (end 111.176 100.899) (width 0.2) (layer "F.Cu") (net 14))
 (segment (start 111.176 100.899) (end 110.575 101.5) (width 0.2) (layer "F.Cu") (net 14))
 (via (at 110.575 101.5) (size 0.6) (drill 0.3) (layers "F.Cu" "B.Cu") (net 14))
 (segment (start 124.5 93.6) (end 126 95.1) (width 0.2) (layer "F.Cu") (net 5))
 (segment (start 126 95.1) (end 126 97.0375) (width 0.2) (layer "F.Cu") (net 5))
 (segment (start 126 97.0375) (end 124.5 98.5375) (width 0.2) (layer "F.Cu") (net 5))
 (via (at 124.5 98.5375) (size 0.6) (drill 0.3) (layers "F.Cu" "B.Cu") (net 5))
 (via (at 124.5 96.4) (size 0.6) (drill 0.3) (layers "F.Cu" "B.Cu") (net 4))
 (segment (start 122.794 82.006) (end 122.794 94.694) (width 0.2) (layer "B.Cu") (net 4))
 (segment (start 122.794 94.694) (end 124.5 96.4) (width 0.2) (layer "B.Cu") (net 4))
 (segment (start 125.975 78.825) (end 122.794 82.006) (width 0.2) (layer "B.Cu") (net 4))
 (segment (start 112.04 102.96) (end 113.5 101.5) (width 0.2) (layer "F.Cu") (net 1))
 (segment (start 127.6 97.54) (end 127.6 98.3625) (width 0.2) (layer "F.Cu") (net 1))
 (segment (start 107.5 97.77384) (end 106.34 96.61384) (width 0.2) (layer "F.Cu") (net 1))
 (segment (start 127.6 98.3625) (end 124.5 101.4625) (width 0.2) (layer "F.Cu") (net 1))
 (segment (start 107.5 102.96) (end 107.5 97.77384) (width 0.2) (layer "F.Cu") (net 1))
 (segment (start 107.5 102.96) (end 112.04 102.96) (width 0.2) (layer "F.Cu") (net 1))
 (segment (start 106.34 96.61384) (end 106.34 90.88) (width 0.2) (layer "F.Cu") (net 1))
 (via (at 124.5 101.4625) (size 0.6) (drill 0.3) (layers "F.Cu" "B.Cu") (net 1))
 (via (at 113.5 101.5) (size 0.6) (drill 0.3) (layers "F.Cu" "B.Cu") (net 1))
 (segment (start 106.34 83.12) (end 106.34 90.88) (width 0.2) (layer "B.Cu") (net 1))
 (segment (start 107.72 89.5) (end 111.9625 89.5) (width 0.2) (layer "B.Cu") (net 1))
 (segment (start 107.5 81.96) (end 106.34 83.12) (width 0.2) (layer "B.Cu") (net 1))
 (segment (start 113.5375 101.4625) (end 113.5 101.5) (width 0.2) (layer "B.Cu") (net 1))
 (segment (start 106.34 90.88) (end 107.72 89.5) (width 0.2) (layer "B.Cu") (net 1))
 (segment (start 111.9625 89.5) (end 113.4625 88) (width 0.2) (layer "B.Cu") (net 1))
 (segment (start 124.5 101.4625) (end 113.5375 101.4625) (width 0.2) (layer "B.Cu") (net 1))
 (segment (start 108.88 98.5) (end 109.981 97.399) (width 0.2) (layer "F.Cu") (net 9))
 (segment (start 112.521 97.399) (end 119.04 90.88) (width 0.2) (layer "F.Cu") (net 9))
 (segment (start 109.981 97.399) (end 112.521 97.399) (width 0.2) (layer "F.Cu") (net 9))
 (segment (start 108.88 98.5) (end 108.88 104) (width 0.2) (layer "B.Cu") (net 9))
 (segment (start 121.9925 104) (end 108.88 104) (width 0.2) (layer "B.Cu") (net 9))
 (segment (start 122.7925 104.8) (end 121.9925 104) (width 0.2) (layer "B.Cu") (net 9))
 (segment (start 108.88 104) (end 108.88 104.12) (width 0.2) (layer "B.Cu") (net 9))
 (segment (start 108.88 104.12) (end 107.5 105.5) (width 0.2) (layer "B.Cu") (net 9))
 (segment (start 115.9215 84.974) (end 116.1475 85.2) (width 0.2) (layer "F.Cu") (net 3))
 (segment (start 114.106 105.974) (end 121.58 98.5) (width 0.2) (layer "F.Cu") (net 3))
 (segment (start 127.6 92.46) (end 128.751 93.611) (width 0.2) (layer "F.Cu") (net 3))
 (segment (start 109.566 84.974) (end 115.9215 84.974) (width 0.2) (layer "F.Cu") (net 3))
 (segment (start 116.7485 84.599) (end 123.169 84.599) (width 0.2) (layer "F.Cu") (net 3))
 (segment (start 109.566 105.974) (end 114.106 105.974) (width 0.2) (layer "F.Cu") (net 3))
 (segment (start 116.1475 85.2) (end 116.7485 84.599) (width 0.2) (layer "F.Cu") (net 3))
 (segment (start 107.5 87.04) (end 109.566 84.974) (width 0.2) (layer "F.Cu") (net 3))
 (segment (start 123.169 84.599) (end 123.695 85.125) (width 0.2) (layer "F.Cu") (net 3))
 (segment (start 107.5 108.04) (end 109.566 105.974) (width 0.2) (layer "F.Cu") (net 3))
 (segment (start 128.751 103.4015) (end 127.3525 104.8) (width 0.2) (layer "F.Cu") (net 3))
 (segment (start 128.751 93.611) (end 128.751 103.4015) (width 0.2) (layer "F.Cu") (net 3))
 (via (at 123.695 85.125) (size 0.6) (drill 0.3) (layers "F.Cu" "B.Cu") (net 3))
 (via (at 116.1475 85.2) (size 0.6) (drill 0.3) (layers "F.Cu" "B.Cu") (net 3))
 (via (at 127.3525 104.8) (size 0.6) (drill 0.3) (layers "F.Cu" "B.Cu") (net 3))
 (segment (start 123.695 88.555) (end 127.6 92.46) (width 0.2) (layer "B.Cu") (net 3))
 (segment (start 124.16216 99.401) (end 122.481 99.401) (width 0.2) (layer "B.Cu") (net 3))
 (segment (start 127.3525 102.59134) (end 124.16216 99.401) (width 0.2) (layer "B.Cu") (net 3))
 (segment (start 123.695 85.125) (end 123.695 88.555) (width 0.2) (layer "B.Cu") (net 3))
 (segment (start 122.481 99.401) (end 121.58 98.5) (width 0.2) (layer "B.Cu") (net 3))
 (segment (start 127.3525 104.8) (end 127.3525 102.59134) (width 0.2) (layer "B.Cu") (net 3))
 (segment (start 120.141 85.7665) (end 120.7075 85.2) (width 0.2) (layer "F.Cu") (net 2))
 (segment (start 116.5 98.5) (end 120.141 94.859) (width 0.2) (layer "F.Cu") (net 2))
 (segment (start 120.141 94.859) (end 120.141 85.7665) (width 0.2) (layer "F.Cu") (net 2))
 (via (at 120.7075 85.2) (size 0.6) (drill 0.3) (layers "F.Cu" "B.Cu") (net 2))
 (segment (start 119.3065 83.799) (end 120.7075 85.2) (width 0.2) (layer "B.Cu") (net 2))
 (segment (start 107.441 97.399) (end 115.399 97.399) (width 0.2) (layer "B.Cu") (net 2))
 (segment (start 107.5 84.5) (end 108.201 83.799) (width 0.2) (layer "B.Cu") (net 2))
 (segment (start 106.34 98.5) (end 107.441 97.399) (width 0.2) (layer "B.Cu") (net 2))
 (segment (start 108.201 83.799) (end 119.3065 83.799) (width 0.2) (layer "B.Cu") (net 2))
 (segment (start 115.399 97.399) (end 116.5 98.5) (width 0.2) (layer "B.Cu") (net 2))
 (segment (start 128.855 85.725) (end 128.855 93.745) (width 0.2) (layer "B.Cu") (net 6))
 (segment (start 128.255 85.125) (end 128.855 85.725) (width 0.2) (layer "B.Cu") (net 6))
 (segment (start 128.855 93.745) (end 127.6 95) (width 0.2) (layer "B.Cu") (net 6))
 (segment (start 120.081 97.001) (end 113.96 90.88) (width 0.2) (layer "B.Cu") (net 6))
 (segment (start 125.599 97.001) (end 120.081 97.001) (width 0.2) (layer "B.Cu") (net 6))
 (segment (start 127.6 95) (end 125.599 97.001) (width 0.2) (layer "B.Cu") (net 6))
 (segment (start 121.58 95.96) (end 121.58 90.88) (width 0.2) (layer "F.Cu") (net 10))
 (segment (start 119.04 98.5) (end 121.58 95.96) (width 0.2) (layer "F.Cu") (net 10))
 (segment (start 117.538 100.002) (end 119.04 98.5) (width 0.2) (layer "B.Cu") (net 10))
 (segment (start 111.42 98.5) (end 112.922 100.002) (width 0.2) (layer "B.Cu") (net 10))
 (segment (start 112.922 100.002) (end 117.538 100.002) (width 0.2) (layer "B.Cu") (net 10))
 (segment (start 115.399 89.779) (end 109.981 89.779) (width 0.2) (layer "F.Cu") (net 12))
 (segment (start 109.981 89.779) (end 108.88 90.88) (width 0.2) (layer "F.Cu") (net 12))
 (segment (start 116.5 90.88) (end 115.399 89.779) (width 0.2) (layer "F.Cu") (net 12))
 (segment (start 115.061 99.601) (end 116.95605 99.601) (width 0.2) (layer "B.Cu") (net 11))
 (segment (start 116.95605 99.601) (end 117.601 98.95605) (width 0.2) (layer "B.Cu") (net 11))
 (segment (start 117.601 98.95605) (end 117.601 97.061) (width 0.2) (layer "B.Cu") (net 11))
 (segment (start 113.96 98.5) (end 115.061 99.601) (width 0.2) (layer "B.Cu") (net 11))
 (segment (start 117.601 97.061) (end 111.42 90.88) (width 0.2) (layer "B.Cu") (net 11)))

